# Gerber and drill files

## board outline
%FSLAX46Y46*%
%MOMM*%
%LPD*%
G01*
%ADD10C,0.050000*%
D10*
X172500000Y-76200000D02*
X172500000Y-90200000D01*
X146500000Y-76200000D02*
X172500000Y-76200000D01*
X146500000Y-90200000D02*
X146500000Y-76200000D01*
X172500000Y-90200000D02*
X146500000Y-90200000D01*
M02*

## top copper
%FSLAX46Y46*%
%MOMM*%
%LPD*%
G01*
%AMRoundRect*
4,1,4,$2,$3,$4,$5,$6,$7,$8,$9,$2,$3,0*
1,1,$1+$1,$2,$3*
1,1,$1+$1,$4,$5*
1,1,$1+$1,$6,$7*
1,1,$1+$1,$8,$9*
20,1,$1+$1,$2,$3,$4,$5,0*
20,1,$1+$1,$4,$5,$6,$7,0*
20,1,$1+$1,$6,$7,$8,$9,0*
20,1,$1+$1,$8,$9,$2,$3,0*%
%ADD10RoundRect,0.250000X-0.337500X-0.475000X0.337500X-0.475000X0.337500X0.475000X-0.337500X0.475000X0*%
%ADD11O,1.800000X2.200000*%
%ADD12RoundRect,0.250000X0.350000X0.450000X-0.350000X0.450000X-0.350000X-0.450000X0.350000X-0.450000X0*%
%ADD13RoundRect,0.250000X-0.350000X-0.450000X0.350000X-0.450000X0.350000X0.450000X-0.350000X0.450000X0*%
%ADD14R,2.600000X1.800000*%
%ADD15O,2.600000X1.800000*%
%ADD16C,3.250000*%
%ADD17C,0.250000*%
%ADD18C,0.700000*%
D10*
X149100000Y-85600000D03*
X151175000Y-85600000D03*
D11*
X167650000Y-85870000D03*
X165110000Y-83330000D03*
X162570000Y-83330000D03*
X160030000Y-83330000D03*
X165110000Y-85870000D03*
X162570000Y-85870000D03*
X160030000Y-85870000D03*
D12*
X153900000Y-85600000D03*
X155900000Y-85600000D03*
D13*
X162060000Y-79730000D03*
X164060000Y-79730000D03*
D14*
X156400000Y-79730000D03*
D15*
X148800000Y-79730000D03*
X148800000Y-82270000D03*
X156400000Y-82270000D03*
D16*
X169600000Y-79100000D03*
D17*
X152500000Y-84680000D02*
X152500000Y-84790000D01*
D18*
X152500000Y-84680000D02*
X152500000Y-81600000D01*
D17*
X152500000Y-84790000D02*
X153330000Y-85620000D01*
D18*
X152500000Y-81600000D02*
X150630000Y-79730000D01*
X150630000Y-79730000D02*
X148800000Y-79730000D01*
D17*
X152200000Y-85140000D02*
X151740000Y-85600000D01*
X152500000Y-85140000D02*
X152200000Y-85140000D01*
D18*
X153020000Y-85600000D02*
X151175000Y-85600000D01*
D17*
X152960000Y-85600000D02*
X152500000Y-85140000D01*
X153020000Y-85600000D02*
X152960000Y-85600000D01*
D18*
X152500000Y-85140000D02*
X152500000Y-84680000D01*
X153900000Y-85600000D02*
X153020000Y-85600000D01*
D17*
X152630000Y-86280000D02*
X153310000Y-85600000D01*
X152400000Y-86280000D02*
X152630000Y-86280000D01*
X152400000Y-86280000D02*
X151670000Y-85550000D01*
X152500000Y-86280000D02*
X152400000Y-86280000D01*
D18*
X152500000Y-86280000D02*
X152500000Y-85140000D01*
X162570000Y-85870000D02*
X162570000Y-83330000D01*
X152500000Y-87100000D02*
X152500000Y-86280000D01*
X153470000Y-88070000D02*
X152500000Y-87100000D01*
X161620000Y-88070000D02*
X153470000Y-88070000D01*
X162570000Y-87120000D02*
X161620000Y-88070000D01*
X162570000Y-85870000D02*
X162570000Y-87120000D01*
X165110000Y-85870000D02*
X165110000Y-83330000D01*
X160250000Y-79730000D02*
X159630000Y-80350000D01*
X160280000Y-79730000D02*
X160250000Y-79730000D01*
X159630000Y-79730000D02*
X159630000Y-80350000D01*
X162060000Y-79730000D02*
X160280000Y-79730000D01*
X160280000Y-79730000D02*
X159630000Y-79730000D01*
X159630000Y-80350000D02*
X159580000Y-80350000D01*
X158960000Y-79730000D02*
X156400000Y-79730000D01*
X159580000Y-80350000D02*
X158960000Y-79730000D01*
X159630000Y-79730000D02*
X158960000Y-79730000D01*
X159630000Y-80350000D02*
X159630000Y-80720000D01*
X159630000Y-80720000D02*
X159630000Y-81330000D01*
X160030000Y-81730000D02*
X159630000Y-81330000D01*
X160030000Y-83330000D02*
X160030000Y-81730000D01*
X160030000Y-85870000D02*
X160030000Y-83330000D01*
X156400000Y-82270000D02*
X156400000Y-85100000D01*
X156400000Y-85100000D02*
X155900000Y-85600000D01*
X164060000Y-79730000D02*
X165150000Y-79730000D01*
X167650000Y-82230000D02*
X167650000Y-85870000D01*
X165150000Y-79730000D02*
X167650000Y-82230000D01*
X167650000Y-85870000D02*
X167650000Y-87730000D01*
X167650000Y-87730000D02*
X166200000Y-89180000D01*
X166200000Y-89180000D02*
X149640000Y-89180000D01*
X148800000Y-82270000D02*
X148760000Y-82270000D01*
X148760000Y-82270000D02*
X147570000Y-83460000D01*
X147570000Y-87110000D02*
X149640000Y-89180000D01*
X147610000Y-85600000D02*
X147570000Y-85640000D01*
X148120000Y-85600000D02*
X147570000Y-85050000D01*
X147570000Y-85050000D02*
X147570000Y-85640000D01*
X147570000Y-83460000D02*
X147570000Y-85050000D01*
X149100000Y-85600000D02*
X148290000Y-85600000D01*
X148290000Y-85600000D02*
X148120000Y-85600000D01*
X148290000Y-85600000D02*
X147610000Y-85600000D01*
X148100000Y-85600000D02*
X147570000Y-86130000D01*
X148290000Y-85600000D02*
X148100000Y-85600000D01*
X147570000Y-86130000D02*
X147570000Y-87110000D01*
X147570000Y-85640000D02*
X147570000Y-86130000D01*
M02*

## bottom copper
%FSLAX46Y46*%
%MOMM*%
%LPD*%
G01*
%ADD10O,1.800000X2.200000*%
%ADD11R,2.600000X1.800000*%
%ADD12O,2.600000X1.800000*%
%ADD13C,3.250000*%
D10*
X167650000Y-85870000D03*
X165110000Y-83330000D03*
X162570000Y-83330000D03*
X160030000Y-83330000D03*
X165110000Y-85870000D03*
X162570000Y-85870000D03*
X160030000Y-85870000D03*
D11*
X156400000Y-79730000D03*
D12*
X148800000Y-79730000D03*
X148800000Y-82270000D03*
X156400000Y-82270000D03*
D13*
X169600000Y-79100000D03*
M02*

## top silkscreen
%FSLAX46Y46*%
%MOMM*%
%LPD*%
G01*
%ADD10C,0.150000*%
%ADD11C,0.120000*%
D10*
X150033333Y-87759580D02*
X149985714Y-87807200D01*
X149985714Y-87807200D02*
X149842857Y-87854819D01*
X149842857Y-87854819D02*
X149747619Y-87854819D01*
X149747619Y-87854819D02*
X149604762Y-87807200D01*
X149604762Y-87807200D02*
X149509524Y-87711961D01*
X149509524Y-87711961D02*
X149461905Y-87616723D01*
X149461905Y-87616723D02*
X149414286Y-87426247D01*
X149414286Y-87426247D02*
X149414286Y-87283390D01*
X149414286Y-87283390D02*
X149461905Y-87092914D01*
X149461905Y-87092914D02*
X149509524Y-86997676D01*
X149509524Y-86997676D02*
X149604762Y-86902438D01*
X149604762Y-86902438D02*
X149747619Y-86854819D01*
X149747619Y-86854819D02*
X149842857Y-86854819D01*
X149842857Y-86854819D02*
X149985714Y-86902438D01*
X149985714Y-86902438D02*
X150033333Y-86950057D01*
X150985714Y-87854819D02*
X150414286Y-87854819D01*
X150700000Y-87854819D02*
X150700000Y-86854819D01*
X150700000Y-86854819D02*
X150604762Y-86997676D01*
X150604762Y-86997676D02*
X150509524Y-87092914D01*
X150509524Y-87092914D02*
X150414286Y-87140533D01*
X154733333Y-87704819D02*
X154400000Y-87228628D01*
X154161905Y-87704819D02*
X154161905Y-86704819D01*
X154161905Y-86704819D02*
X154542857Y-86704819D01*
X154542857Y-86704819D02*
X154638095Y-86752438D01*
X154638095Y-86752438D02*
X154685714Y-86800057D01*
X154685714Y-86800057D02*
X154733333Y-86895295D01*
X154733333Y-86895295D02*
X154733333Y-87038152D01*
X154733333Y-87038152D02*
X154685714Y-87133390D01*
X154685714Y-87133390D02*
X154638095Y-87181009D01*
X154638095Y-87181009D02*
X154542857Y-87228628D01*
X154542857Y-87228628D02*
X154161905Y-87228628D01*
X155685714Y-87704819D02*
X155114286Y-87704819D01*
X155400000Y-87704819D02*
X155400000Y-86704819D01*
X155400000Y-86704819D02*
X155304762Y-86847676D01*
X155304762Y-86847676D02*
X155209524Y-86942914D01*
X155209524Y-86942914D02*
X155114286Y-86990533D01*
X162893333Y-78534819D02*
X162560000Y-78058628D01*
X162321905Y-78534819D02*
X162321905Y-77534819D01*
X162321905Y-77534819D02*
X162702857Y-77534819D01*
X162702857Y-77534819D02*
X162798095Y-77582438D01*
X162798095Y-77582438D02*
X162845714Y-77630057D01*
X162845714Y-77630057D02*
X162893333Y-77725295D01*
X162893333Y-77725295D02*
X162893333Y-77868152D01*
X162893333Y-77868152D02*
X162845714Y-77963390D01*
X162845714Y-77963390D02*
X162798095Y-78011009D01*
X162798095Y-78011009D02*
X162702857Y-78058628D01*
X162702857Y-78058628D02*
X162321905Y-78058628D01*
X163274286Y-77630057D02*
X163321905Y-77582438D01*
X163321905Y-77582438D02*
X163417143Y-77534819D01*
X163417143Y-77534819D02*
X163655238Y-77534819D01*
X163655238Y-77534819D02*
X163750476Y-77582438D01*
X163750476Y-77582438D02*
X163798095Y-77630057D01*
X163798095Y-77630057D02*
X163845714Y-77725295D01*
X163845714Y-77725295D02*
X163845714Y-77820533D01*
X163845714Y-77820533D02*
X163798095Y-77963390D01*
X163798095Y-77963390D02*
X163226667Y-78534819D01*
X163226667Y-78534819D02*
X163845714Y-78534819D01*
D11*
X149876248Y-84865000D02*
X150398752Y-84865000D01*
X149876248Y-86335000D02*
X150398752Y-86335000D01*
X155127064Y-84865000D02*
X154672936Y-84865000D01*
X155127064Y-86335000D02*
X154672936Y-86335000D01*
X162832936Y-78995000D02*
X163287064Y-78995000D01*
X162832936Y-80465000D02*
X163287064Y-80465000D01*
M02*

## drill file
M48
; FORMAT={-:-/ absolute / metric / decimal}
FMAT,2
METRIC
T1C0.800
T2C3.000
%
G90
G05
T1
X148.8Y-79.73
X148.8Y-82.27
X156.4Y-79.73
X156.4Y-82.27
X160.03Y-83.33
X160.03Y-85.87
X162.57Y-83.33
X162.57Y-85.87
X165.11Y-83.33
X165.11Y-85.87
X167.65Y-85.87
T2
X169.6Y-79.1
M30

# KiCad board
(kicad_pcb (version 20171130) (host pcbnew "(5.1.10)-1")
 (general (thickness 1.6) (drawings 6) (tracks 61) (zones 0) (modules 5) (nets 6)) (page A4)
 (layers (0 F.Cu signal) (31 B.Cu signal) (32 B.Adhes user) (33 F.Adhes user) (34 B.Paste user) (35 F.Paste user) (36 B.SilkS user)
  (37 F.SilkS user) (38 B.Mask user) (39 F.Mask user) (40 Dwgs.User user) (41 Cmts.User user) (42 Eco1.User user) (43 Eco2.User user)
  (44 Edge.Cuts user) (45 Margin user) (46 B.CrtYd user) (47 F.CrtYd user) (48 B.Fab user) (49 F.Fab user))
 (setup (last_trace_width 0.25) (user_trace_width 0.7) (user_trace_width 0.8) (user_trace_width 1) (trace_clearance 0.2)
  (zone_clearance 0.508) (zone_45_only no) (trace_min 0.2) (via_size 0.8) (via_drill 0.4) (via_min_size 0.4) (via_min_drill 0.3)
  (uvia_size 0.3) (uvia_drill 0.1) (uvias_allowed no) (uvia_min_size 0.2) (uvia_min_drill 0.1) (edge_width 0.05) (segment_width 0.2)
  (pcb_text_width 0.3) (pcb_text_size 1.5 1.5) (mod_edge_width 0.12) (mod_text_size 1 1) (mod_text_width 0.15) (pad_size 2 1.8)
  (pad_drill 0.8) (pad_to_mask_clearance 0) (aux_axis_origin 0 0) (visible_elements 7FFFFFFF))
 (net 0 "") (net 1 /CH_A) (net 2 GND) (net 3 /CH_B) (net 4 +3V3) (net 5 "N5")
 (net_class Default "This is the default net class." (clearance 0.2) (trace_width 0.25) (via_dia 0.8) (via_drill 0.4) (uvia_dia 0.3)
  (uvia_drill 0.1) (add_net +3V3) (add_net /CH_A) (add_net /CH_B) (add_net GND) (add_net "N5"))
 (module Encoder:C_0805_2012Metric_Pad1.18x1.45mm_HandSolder (layer F.Cu) (at 150.1375 85.6)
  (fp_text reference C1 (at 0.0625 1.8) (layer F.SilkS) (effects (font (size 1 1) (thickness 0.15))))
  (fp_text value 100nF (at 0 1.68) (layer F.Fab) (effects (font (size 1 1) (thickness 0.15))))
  (fp_line (start -0.261252 -0.735) (end 0.261252 -0.735) (layer F.SilkS) (width 0.12))
  (fp_line (start -0.261252 0.735) (end 0.261252 0.735) (layer F.SilkS) (width 0.12))
  (pad 1 smd roundrect (at -1.0375 0) (size 1.175 1.45) (layers F.Cu F.Paste F.Mask) (roundrect_rratio 0.212766) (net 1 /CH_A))
  (pad 2 smd roundrect (at 1.0375 0) (size 1.175 1.45) (layers F.Cu F.Paste F.Mask) (roundrect_rratio 0.212766) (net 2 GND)))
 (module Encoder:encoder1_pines (layer B.Cu) (at 165.11 80.79 180)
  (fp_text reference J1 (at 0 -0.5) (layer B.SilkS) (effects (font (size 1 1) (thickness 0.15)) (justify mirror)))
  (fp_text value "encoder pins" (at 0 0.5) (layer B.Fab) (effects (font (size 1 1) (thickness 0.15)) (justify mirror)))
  (pad 1 thru_hole oval (at -2.54 -5.08 90) (size 2.2 1.8) (drill 0.8) (layers *.Cu *.Mask) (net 1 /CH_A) (solder_mask_margin 0.102))
  (pad 2 thru_hole oval (at 0 -2.54 90) (size 2.2 1.8) (drill 0.8) (layers *.Cu *.Mask) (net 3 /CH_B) (solder_mask_margin 0.102))
  (pad 3 thru_hole oval (at 2.54 -2.54 90) (size 2.2 1.8) (drill 0.8) (layers *.Cu *.Mask) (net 2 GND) (solder_mask_margin 0.102))
  (pad 4 thru_hole oval (at 5.08 -2.54 90) (size 2.2 1.8) (drill 0.8) (layers *.Cu *.Mask) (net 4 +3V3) (solder_mask_margin 0.102))
  (pad 2 thru_hole oval (at 0 -5.08 90) (size 2.2 1.8) (drill 0.8) (layers *.Cu *.Mask) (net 3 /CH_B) (solder_mask_margin 0.102))
  (pad 3 thru_hole oval (at 2.54 -5.08 90) (size 2.2 1.8) (drill 0.8) (layers *.Cu *.Mask) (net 2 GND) (solder_mask_margin 0.102))
  (pad 4 thru_hole oval (at 5.08 -5.08 90) (size 2.2 1.8) (drill 0.8) (layers *.Cu *.Mask) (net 4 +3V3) (solder_mask_margin 0.102)))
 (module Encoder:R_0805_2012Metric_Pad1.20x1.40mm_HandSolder (layer F.Cu) (at 154.9 85.6 180)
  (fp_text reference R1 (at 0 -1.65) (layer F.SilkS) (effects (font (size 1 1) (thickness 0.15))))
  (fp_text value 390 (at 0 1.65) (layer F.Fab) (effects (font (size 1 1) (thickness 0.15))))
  (fp_line (start -0.227064 0.735) (end 0.227064 0.735) (layer F.SilkS) (width 0.12))
  (fp_line (start -0.227064 -0.735) (end 0.227064 -0.735) (layer F.SilkS) (width 0.12))
  (pad 2 smd roundrect (at 1 0 180) (size 1.2 1.4) (layers F.Cu F.Paste F.Mask) (roundrect_rratio 0.208333) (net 2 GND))
  (pad 1 smd roundrect (at -1 0 180) (size 1.2 1.4) (layers F.Cu F.Paste F.Mask) (roundrect_rratio 0.208333) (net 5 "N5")))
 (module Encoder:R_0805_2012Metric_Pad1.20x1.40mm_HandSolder (layer F.Cu) (at 163.06 79.73)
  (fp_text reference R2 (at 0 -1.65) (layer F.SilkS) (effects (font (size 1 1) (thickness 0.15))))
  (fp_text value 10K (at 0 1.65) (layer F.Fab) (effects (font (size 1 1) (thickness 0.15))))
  (fp_line (start -0.227064 -0.735) (end 0.227064 -0.735) (layer F.SilkS) (width 0.12))
  (fp_line (start -0.227064 0.735) (end 0.227064 0.735) (layer F.SilkS) (width 0.12))
  (pad 1 smd roundrect (at -1 0) (size 1.2 1.4) (layers F.Cu F.Paste F.Mask) (roundrect_rratio 0.208333) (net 4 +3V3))
  (pad 2 smd roundrect (at 1 0) (size 1.2 1.4) (layers F.Cu F.Paste F.Mask) (roundrect_rratio 0.208333) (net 1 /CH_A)))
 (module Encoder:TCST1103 (layer B.Cu) (at 152.6 81 180)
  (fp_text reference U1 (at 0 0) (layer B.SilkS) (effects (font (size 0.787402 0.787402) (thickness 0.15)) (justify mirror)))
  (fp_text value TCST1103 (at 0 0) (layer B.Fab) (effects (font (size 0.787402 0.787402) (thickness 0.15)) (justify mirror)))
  (pad 1 thru_hole rect (at -3.8 1.27 180) (size 2.6 1.8) (drill 0.8) (layers *.Cu *.Mask) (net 4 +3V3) (solder_mask_margin 0.102))
  (pad 3 thru_hole oval (at 3.8 1.27 180) (size 2.6 1.8) (drill 0.8) (layers *.Cu *.Mask) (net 2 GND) (solder_mask_margin 0.102))
  (pad 4 thru_hole oval (at 3.8 -1.27 180) (size 2.6 1.8) (drill 0.8) (layers *.Cu *.Mask) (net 1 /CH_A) (solder_mask_margin 0.102))
  (pad 2 thru_hole oval (at -3.8 -1.27 180) (size 2.6 1.8) (drill 0.8) (layers *.Cu *.Mask) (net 5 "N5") (solder_mask_margin 0.102)))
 (gr_line (start 172.5 76.2) (end 172.5 90.2) (layer Edge.Cuts) (width 0.05))
 (gr_line (start 146.5 76.2) (end 172.5 76.2) (layer Edge.Cuts) (width 0.05))
 (gr_line (start 146.5 90.2) (end 146.5 76.2) (layer Edge.Cuts) (width 0.05))
 (gr_line (start 172.5 90.2) (end 146.5 90.2) (layer Edge.Cuts) (width 0.05))
 (via (at 169.6 79.1) (size 3.25) (drill 3) (layers F.Cu B.Cu) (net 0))
 (segment (start 152.5 84.68) (end 152.5 84.79) (width 0.25) (layer F.Cu) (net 2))
 (segment (start 152.5 84.68) (end 152.5 81.6) (width 0.7) (layer F.Cu) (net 2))
 (segment (start 152.5 84.79) (end 153.33 85.62) (width 0.25) (layer F.Cu) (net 2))
 (segment (start 152.5 81.6) (end 150.63 79.73) (width 0.7) (layer F.Cu) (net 2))
 (segment (start 150.63 79.73) (end 148.8 79.73) (width 0.7) (layer F.Cu) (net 2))
 (segment (start 152.2 85.14) (end 151.74 85.6) (width 0.25) (layer F.Cu) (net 2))
 (segment (start 152.5 85.14) (end 152.2 85.14) (width 0.25) (layer F.Cu) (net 2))
 (segment (start 153.02 85.6) (end 151.175 85.6) (width 0.7) (layer F.Cu) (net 2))
 (segment (start 152.96 85.6) (end 152.5 85.14) (width 0.25) (layer F.Cu) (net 2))
 (segment (start 153.02 85.6) (end 152.96 85.6) (width 0.25) (layer F.Cu) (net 2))
 (segment (start 152.5 85.14) (end 152.5 84.68) (width 0.7) (layer F.Cu) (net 2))
 (segment (start 153.9 85.6) (end 153.02 85.6) (width 0.7) (layer F.Cu) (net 2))
 (segment (start 152.63 86.28) (end 153.31 85.6) (width 0.25) (layer F.Cu) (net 2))
 (segment (start 152.4 86.28) (end 152.63 86.28) (width 0.25) (layer F.Cu) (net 2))
 (segment (start 152.4 86.28) (end 151.67 85.55) (width 0.25) (layer F.Cu) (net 2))
 (segment (start 152.5 86.28) (end 152.4 86.28) (width 0.25) (layer F.Cu) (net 2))
 (segment (start 152.5 86.28) (end 152.5 85.14) (width 0.7) (layer F.Cu) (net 2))
 (segment (start 162.57 85.87) (end 162.57 83.33) (width 0.7) (layer F.Cu) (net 2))
 (segment (start 152.5 87.1) (end 152.5 86.28) (width 0.7) (layer F.Cu) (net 2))
 (segment (start 153.47 88.07) (end 152.5 87.1) (width 0.7) (layer F.Cu) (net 2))
 (segment (start 161.62 88.07) (end 153.47 88.07) (width 0.7) (layer F.Cu) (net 2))
 (segment (start 162.57 87.12) (end 161.62 88.07) (width 0.7) (layer F.Cu) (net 2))
 (segment (start 162.57 85.87) (end 162.57 87.12) (width 0.7) (layer F.Cu) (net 2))
 (segment (start 165.11 85.87) (end 165.11 83.33) (width 0.7) (layer F.Cu) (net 3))
 (segment (start 160.25 79.73) (end 159.63 80.35) (width 0.7) (layer F.Cu) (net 4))
 (segment (start 160.28 79.73) (end 160.25 79.73) (width 0.7) (layer F.Cu) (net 4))
 (segment (start 159.63 79.73) (end 159.63 80.35) (width 0.7) (layer F.Cu) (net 4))
 (segment (start 162.06 79.73) (end 160.28 79.73) (width 0.7) (layer F.Cu) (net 4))
 (segment (start 160.28 79.73) (end 159.63 79.73) (width 0.7) (layer F.Cu) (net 4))
 (segment (start 159.63 80.35) (end 159.58 80.35) (width 0.7) (layer F.Cu) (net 4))
 (segment (start 158.96 79.73) (end 156.4 79.73) (width 0.7) (layer F.Cu) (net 4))
 (segment (start 159.58 80.35) (end 158.96 79.73) (width 0.7) (layer F.Cu) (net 4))
 (segment (start 159.63 79.73) (end 158.96 79.73) (width 0.7) (layer F.Cu) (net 4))
 (segment (start 159.63 80.35) (end 159.63 80.72) (width 0.7) (layer F.Cu) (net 4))
 (segment (start 159.63 80.72) (end 159.63 81.33) (width 0.7) (layer F.Cu) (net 4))
 (segment (start 160.03 81.73) (end 159.63 81.33) (width 0.7) (layer F.Cu) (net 4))
 (segment (start 160.03 83.33) (end 160.03 81.73) (width 0.7) (layer F.Cu) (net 4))
 (segment (start 160.03 85.87) (end 160.03 83.33) (width 0.7) (layer F.Cu) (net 4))
 (segment (start 156.4 82.27) (end 156.4 85.1) (width 0.7) (layer F.Cu) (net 5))
 (segment (start 156.4 85.1) (end 155.9 85.6) (width 0.7) (layer F.Cu) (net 5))
 (segment (start 164.06 79.73) (end 165.15 79.73) (width 0.7) (layer F.Cu) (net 1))
 (segment (start 167.65 82.23) (end 167.65 85.87) (width 0.7) (layer F.Cu) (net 1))
 (segment (start 165.15 79.73) (end 167.65 82.23) (width 0.7) (layer F.Cu) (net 1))
 (segment (start 167.65 85.87) (end 167.65 87.73) (width 0.7) (layer F.Cu) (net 1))
 (segment (start 167.65 87.73) (end 166.2 89.18) (width 0.7) (layer F.Cu) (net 1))
 (segment (start 166.2 89.18) (end 149.64 89.18) (width 0.7) (layer F.Cu) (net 1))
 (segment (start 148.8 82.27) (end 148.76 82.27) (width 0.7) (layer F.Cu) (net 1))
 (segment (start 148.76 82.27) (end 147.57 83.46) (width 0.7) (layer F.Cu) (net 1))
 (segment (start 147.57 87.11) (end 149.64 89.18) (width 0.7) (layer F.Cu) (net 1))
 (segment (start 147.61 85.6) (end 147.57 85.64) (width 0.7) (layer F.Cu) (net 1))
 (segment (start 148.12 85.6) (end 147.57 85.05) (width 0.7) (layer F.Cu) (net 1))
 (segment (start 147.57 85.05) (end 147.57 85.64) (width 0.7) (layer F.Cu) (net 1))
 (segment (start 147.57 83.46) (end 147.57 85.05) (width 0.7) (layer F.Cu) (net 1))
 (segment (start 149.1 85.6) (end 148.29 85.6) (width 0.7) (layer F.Cu) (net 1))
 (segment (start 148.29 85.6) (end 148.12 85.6) (width 0.7) (layer F.Cu) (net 1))
 (segment (start 148.29 85.6) (end 147.61 85.6) (width 0.7) (layer F.Cu) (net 1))
 (segment (start 148.1 85.6) (end 147.57 86.13) (width 0.7) (layer F.Cu) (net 1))
 (segment (start 148.29 85.6) (end 148.1 85.6) (width 0.7) (layer F.Cu) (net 1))
 (segment (start 147.57 86.13) (end 147.57 87.11) (width 0.7) (layer F.Cu) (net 1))
 (segment (start 147.57 85.64) (end 147.57 86.13) (width 0.7) (layer F.Cu) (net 1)))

